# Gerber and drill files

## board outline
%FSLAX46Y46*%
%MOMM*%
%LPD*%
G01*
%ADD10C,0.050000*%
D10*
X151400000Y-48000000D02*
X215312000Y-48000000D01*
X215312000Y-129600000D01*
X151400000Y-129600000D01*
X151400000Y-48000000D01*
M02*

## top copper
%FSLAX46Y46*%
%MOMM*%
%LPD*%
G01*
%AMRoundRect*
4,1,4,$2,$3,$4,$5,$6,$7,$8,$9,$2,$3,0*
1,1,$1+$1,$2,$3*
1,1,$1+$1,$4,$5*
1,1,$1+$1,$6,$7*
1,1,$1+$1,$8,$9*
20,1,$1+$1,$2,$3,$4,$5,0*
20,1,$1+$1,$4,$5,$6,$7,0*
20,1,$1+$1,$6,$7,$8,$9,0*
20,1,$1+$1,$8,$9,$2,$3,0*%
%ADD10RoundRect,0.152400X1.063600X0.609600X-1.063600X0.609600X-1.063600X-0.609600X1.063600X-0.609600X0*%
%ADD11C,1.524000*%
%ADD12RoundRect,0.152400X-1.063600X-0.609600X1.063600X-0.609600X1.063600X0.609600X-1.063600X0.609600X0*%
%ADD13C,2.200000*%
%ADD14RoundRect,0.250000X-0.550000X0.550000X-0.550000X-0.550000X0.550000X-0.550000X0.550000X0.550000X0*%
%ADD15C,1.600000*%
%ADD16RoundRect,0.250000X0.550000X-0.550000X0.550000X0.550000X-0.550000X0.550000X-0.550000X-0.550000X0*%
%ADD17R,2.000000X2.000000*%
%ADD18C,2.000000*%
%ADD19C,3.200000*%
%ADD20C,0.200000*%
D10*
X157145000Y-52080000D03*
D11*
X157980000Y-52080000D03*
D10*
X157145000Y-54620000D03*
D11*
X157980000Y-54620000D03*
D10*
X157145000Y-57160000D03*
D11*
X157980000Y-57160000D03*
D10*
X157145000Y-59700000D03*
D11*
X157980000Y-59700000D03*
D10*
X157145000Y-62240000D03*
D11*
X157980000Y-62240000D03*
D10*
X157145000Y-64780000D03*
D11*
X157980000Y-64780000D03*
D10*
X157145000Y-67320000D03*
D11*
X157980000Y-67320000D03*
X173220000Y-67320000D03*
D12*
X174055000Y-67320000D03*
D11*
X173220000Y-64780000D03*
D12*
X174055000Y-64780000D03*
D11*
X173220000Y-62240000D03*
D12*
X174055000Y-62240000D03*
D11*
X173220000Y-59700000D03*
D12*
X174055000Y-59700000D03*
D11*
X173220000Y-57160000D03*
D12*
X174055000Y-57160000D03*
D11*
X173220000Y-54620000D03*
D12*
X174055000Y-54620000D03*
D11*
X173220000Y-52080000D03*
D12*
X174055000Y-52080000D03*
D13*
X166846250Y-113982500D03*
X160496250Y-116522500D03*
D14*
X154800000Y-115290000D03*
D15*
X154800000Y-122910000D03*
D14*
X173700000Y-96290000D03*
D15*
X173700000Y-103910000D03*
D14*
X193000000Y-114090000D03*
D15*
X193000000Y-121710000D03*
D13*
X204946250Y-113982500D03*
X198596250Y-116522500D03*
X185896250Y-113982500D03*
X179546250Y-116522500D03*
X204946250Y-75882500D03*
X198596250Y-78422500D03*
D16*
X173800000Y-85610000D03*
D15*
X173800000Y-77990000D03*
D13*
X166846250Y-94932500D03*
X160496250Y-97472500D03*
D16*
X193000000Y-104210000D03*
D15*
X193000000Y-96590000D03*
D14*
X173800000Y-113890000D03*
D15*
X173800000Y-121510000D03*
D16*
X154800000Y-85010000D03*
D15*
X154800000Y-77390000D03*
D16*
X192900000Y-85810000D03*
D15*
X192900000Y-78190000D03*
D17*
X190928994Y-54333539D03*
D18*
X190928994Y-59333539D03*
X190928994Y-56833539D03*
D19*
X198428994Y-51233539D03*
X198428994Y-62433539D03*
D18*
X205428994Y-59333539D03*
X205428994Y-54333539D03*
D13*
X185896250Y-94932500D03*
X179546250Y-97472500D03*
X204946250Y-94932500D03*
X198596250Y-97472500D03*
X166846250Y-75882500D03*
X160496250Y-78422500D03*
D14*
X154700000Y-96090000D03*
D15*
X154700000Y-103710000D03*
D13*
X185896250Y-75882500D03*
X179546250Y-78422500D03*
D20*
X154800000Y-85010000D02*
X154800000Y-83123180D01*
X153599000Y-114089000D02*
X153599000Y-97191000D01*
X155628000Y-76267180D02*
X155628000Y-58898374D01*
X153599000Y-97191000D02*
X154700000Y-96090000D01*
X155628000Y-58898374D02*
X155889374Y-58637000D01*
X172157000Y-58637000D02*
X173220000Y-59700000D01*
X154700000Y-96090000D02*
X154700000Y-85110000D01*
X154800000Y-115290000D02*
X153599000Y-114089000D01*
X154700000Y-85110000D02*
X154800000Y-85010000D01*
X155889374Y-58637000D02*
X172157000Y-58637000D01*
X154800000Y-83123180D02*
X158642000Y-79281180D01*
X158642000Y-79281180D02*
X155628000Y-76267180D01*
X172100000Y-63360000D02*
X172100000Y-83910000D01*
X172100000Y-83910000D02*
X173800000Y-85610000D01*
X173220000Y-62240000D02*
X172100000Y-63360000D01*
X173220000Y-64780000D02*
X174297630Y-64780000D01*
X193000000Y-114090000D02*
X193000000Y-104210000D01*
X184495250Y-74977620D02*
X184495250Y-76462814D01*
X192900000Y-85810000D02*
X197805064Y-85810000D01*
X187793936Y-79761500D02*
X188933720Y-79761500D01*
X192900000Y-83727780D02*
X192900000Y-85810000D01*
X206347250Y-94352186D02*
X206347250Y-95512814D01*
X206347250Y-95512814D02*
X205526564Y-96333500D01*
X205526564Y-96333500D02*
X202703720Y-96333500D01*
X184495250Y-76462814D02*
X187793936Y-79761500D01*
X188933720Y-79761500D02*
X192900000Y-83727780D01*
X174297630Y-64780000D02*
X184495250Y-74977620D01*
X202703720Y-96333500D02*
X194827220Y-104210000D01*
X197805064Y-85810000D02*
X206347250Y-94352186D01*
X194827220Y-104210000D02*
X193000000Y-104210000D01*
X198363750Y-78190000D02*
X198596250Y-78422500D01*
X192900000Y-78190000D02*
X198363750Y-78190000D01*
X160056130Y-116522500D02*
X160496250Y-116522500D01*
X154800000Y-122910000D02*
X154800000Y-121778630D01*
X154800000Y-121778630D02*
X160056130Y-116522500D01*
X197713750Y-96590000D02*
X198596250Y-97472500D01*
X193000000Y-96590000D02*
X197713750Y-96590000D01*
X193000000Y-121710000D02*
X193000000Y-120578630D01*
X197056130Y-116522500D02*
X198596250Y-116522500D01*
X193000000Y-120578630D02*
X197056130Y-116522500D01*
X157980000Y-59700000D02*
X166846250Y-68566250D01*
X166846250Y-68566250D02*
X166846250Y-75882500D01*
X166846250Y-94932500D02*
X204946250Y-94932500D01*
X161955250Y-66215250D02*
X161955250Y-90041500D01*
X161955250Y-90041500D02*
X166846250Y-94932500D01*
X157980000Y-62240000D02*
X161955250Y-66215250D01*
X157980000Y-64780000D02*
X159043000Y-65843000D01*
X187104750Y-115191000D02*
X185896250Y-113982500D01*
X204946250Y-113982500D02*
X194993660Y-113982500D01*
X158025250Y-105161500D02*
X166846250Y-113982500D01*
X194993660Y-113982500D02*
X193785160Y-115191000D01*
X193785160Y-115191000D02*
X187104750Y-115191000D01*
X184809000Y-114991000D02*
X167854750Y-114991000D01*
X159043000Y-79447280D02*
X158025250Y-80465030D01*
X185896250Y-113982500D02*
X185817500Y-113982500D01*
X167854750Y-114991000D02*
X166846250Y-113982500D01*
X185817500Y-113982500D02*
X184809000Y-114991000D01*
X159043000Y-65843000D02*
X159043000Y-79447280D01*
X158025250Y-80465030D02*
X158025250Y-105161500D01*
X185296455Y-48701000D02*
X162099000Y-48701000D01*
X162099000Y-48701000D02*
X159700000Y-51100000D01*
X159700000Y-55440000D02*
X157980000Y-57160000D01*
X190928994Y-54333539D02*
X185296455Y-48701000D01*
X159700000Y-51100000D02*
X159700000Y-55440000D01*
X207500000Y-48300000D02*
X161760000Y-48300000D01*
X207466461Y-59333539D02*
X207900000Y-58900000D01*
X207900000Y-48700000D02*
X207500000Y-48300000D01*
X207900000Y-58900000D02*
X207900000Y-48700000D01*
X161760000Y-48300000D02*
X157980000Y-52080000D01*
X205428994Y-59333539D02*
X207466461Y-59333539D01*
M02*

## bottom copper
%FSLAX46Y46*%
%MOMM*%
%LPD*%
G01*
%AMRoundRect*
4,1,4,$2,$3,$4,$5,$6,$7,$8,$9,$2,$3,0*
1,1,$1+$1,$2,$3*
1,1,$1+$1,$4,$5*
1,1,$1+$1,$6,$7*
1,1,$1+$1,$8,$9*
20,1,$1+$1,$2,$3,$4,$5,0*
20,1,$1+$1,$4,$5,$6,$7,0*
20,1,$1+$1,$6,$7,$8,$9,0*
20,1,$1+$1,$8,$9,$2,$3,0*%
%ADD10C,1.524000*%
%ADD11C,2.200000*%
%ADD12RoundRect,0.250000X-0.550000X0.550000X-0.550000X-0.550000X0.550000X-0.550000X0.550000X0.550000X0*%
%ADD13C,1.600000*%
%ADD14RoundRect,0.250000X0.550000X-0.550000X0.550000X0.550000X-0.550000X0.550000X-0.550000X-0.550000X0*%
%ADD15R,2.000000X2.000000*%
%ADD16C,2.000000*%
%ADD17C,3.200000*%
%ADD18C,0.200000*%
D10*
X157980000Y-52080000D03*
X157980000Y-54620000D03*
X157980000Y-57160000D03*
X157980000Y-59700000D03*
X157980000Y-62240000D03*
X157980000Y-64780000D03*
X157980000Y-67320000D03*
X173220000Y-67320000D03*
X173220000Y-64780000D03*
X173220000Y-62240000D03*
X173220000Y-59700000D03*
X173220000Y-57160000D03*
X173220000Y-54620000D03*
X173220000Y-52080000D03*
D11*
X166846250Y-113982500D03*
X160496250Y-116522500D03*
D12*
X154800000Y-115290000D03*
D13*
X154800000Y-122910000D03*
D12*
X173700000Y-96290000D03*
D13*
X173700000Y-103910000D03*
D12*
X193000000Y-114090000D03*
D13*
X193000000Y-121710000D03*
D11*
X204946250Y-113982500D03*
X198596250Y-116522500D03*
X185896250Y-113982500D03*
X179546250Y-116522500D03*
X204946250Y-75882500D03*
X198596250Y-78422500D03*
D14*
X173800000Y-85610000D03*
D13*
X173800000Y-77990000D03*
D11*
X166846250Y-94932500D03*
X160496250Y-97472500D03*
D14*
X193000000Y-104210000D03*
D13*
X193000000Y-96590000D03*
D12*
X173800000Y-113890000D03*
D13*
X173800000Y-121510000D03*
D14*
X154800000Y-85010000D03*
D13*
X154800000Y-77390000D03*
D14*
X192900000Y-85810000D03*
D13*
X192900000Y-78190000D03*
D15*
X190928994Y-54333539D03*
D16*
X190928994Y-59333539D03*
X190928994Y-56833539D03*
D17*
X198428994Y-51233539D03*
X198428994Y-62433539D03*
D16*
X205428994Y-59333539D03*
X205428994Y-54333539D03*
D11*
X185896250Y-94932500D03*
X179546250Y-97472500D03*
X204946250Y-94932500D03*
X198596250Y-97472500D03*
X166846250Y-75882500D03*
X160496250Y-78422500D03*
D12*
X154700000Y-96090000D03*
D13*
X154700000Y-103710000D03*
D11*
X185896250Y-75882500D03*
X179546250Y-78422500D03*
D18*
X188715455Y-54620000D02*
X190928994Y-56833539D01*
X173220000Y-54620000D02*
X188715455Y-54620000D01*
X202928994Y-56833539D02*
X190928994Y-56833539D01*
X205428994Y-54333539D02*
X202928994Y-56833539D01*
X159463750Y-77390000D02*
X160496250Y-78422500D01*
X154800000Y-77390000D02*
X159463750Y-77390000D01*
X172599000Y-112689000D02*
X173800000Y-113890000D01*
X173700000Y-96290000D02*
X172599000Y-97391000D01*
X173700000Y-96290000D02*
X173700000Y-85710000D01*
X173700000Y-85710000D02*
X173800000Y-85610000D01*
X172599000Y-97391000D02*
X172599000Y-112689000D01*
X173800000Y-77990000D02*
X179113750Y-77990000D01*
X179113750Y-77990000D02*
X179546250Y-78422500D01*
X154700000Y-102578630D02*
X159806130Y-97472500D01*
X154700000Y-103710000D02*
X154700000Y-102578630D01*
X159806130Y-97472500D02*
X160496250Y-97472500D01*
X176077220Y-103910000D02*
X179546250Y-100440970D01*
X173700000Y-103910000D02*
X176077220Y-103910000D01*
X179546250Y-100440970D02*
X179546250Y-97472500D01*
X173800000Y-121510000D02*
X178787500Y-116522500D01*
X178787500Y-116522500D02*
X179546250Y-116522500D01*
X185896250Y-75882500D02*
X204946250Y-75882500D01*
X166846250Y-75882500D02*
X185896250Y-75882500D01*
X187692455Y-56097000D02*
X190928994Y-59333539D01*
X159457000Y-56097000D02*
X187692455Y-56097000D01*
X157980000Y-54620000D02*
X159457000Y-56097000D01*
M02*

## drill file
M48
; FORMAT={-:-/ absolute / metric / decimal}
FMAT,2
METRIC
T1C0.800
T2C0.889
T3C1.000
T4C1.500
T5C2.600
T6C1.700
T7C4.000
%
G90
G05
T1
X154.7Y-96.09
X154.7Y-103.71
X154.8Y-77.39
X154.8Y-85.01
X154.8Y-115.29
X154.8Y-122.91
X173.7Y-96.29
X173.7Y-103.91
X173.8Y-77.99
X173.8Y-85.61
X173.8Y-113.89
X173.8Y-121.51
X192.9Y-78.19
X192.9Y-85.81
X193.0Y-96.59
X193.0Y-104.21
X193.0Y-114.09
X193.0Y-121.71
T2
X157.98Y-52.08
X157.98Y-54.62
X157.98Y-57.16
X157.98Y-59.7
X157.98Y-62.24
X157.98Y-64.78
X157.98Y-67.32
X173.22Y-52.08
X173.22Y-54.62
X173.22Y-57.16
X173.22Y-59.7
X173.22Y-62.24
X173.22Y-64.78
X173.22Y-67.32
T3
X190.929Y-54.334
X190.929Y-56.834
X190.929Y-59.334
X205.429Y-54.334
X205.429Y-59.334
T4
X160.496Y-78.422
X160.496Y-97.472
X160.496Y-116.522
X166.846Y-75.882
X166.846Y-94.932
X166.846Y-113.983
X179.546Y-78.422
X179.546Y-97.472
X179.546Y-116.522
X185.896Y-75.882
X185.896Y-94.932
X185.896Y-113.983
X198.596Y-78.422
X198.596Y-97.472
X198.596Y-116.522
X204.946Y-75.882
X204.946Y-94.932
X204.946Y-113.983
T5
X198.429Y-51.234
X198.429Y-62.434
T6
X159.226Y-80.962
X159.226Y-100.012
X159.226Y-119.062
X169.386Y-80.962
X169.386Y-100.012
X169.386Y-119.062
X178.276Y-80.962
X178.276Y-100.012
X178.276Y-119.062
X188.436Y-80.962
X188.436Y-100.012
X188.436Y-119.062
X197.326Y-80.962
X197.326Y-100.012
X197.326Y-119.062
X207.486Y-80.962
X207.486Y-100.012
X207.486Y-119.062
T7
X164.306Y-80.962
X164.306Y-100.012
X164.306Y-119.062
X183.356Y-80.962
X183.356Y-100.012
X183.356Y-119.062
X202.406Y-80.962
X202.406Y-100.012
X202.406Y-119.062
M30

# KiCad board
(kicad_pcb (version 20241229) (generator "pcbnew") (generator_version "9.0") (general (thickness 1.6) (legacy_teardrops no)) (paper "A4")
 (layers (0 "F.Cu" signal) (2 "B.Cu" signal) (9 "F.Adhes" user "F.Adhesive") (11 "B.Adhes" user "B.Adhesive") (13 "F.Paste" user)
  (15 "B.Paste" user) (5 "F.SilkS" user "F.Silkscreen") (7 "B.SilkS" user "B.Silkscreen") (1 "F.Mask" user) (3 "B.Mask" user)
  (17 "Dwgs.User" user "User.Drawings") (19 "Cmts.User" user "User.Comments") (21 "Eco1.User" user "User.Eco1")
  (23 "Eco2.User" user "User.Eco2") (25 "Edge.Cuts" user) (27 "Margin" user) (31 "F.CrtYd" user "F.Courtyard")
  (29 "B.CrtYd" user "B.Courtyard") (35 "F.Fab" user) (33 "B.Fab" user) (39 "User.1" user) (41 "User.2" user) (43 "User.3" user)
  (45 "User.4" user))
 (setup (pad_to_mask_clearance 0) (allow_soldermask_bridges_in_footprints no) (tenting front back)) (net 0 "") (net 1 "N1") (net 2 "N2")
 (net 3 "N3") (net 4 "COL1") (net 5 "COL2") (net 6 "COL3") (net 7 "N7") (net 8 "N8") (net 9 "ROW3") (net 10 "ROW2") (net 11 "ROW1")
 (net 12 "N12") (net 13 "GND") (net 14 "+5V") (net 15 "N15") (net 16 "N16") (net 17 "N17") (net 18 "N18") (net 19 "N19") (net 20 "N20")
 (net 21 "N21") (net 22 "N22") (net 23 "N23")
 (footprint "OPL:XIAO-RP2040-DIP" (layer "F.Cu") (at 165.6 59.7)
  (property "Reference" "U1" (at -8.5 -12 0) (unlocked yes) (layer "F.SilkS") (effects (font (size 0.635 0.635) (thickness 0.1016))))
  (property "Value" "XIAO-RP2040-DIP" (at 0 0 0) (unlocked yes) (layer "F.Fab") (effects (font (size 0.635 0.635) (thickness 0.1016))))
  (pad "1" smd roundrect (at -8.455 -7.62 180) (size 2.432 1.524) (layers "F.Cu" "F.Mask") (roundrect_rratio 0.1) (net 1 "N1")
   (thermal_bridge_angle 45))
  (pad "1" thru_hole circle (at -7.62 -7.62 180) (size 1.524 1.524) (drill 0.889) (layers "*.Cu" "*.Mask") (remove_unused_layers no)
   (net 1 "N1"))
  (pad "2" smd roundrect (at -8.455 -5.08 180) (size 2.432 1.524) (layers "F.Cu" "F.Mask") (roundrect_rratio 0.1) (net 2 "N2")
   (thermal_bridge_angle 45))
  (pad "2" thru_hole circle (at -7.62 -5.08 180) (size 1.524 1.524) (drill 0.889) (layers "*.Cu" "*.Mask") (remove_unused_layers no)
   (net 2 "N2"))
  (pad "3" smd roundrect (at -8.455 -2.54 180) (size 2.432 1.524) (layers "F.Cu" "F.Mask") (roundrect_rratio 0.1) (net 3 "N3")
   (thermal_bridge_angle 45))
  (pad "3" thru_hole circle (at -7.62 -2.54 180) (size 1.524 1.524) (drill 0.889) (layers "*.Cu" "*.Mask") (remove_unused_layers no)
   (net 3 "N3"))
  (pad "4" smd roundrect (at -8.455 0 180) (size 2.432 1.524) (layers "F.Cu" "F.Mask") (roundrect_rratio 0.1) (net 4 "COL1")
   (thermal_bridge_angle 45))
  (pad "4" thru_hole circle (at -7.62 0 180) (size 1.524 1.524) (drill 0.889) (layers "*.Cu" "*.Mask") (remove_unused_layers no)
   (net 4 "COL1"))
  (pad "5" smd roundrect (at -8.455 2.54 180) (size 2.432 1.524) (layers "F.Cu" "F.Mask") (roundrect_rratio 0.1) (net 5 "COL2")
   (thermal_bridge_angle 45))
  (pad "5" thru_hole circle (at -7.62 2.54 180) (size 1.524 1.524) (drill 0.889) (layers "*.Cu" "*.Mask") (remove_unused_layers no)
   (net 5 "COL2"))
  (pad "6" smd roundrect (at -8.455 5.08 180) (size 2.432 1.524) (layers "F.Cu" "F.Mask") (roundrect_rratio 0.1) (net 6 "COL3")
   (thermal_bridge_angle 45))
  (pad "6" thru_hole circle (at -7.62 5.08 180) (size 1.524 1.524) (drill 0.889) (layers "*.Cu" "*.Mask") (remove_unused_layers no)
   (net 6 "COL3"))
  (pad "7" smd roundrect (at -8.455 7.62 180) (size 2.432 1.524) (layers "F.Cu" "F.Mask") (roundrect_rratio 0.1) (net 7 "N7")
   (thermal_bridge_angle 45))
  (pad "7" thru_hole circle (at -7.62 7.62 180) (size 1.524 1.524) (drill 0.889) (layers "*.Cu" "*.Mask") (remove_unused_layers no)
   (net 7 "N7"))
  (pad "8" thru_hole circle (at 7.62 7.62) (size 1.524 1.524) (drill 0.889) (layers "*.Cu" "*.Mask") (remove_unused_layers no) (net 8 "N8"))
  (pad "8" smd roundrect (at 8.455 7.62) (size 2.432 1.524) (layers "F.Cu" "F.Mask") (roundrect_rratio 0.1) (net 8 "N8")
   (thermal_bridge_angle 45))
  (pad "9" thru_hole circle (at 7.62 5.08) (size 1.524 1.524) (drill 0.889) (layers "*.Cu" "*.Mask") (remove_unused_layers no)
   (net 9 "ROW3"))
  (pad "9" smd roundrect (at 8.455 5.08) (size 2.432 1.524) (layers "F.Cu" "F.Mask") (roundrect_rratio 0.1) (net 9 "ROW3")
   (thermal_bridge_angle 45))
  (pad "10" thru_hole circle (at 7.62 2.54) (size 1.524 1.524) (drill 0.889) (layers "*.Cu" "*.Mask") (remove_unused_layers no)
   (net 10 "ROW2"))
  (pad "10" smd roundrect (at 8.455 2.54) (size 2.432 1.524) (layers "F.Cu" "F.Mask") (roundrect_rratio 0.1) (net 10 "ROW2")
   (thermal_bridge_angle 45))
  (pad "11" thru_hole circle (at 7.62 0) (size 1.524 1.524) (drill 0.889) (layers "*.Cu" "*.Mask") (remove_unused_layers no) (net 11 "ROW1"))
  (pad "11" smd roundrect (at 8.455 0) (size 2.432 1.524) (layers "F.Cu" "F.Mask") (roundrect_rratio 0.1) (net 11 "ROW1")
   (thermal_bridge_angle 45))
  (pad "12" thru_hole circle (at 7.62 -2.54) (size 1.524 1.524) (drill 0.889) (layers "*.Cu" "*.Mask") (remove_unused_layers no)
   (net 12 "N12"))
  (pad "12" smd roundrect (at 8.455 -2.54) (size 2.432 1.524) (layers "F.Cu" "F.Mask") (roundrect_rratio 0.1) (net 12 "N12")
   (thermal_bridge_angle 45))
  (pad "13" thru_hole circle (at 7.62 -5.08) (size 1.524 1.524) (drill 0.889) (layers "*.Cu" "*.Mask") (remove_unused_layers no)
   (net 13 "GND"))
  (pad "13" smd roundrect (at 8.455 -5.08) (size 2.432 1.524) (layers "F.Cu" "F.Mask") (roundrect_rratio 0.1) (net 13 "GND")
   (thermal_bridge_angle 45))
  (pad "14" thru_hole circle (at 7.62 -7.62) (size 1.524 1.524) (drill 0.889) (layers "*.Cu" "*.Mask") (remove_unused_layers no)
   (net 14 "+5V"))
  (pad "14" smd roundrect (at 8.455 -7.62) (size 2.432 1.524) (layers "F.Cu" "F.Mask") (roundrect_rratio 0.1) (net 14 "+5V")
   (thermal_bridge_angle 45)))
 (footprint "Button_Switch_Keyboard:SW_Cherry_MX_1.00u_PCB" (layer "F.Cu") (at 166.84625 113.9825)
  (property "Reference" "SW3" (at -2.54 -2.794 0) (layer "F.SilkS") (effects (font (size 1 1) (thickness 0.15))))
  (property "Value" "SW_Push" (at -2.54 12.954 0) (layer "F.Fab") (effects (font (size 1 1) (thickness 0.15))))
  (pad "" np_thru_hole circle (at -7.62 5.08) (size 1.7 1.7) (drill 1.7) (layers "*.Cu" "*.Mask"))
  (pad "" np_thru_hole circle (at -2.54 5.08) (size 4 4) (drill 4) (layers "*.Cu" "*.Mask"))
  (pad "" np_thru_hole circle (at 2.54 5.08) (size 1.7 1.7) (drill 1.7) (layers "*.Cu" "*.Mask"))
  (pad "1" thru_hole circle (at 0 0) (size 2.2 2.2) (drill 1.5) (layers "*.Cu" "*.Mask") (remove_unused_layers no) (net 6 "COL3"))
  (pad "2" thru_hole circle (at -6.35 2.54) (size 2.2 2.2) (drill 1.5) (layers "*.Cu" "*.Mask") (remove_unused_layers no) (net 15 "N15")))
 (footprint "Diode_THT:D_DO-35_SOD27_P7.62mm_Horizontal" (layer "F.Cu") (at 154.8 115.29 -90)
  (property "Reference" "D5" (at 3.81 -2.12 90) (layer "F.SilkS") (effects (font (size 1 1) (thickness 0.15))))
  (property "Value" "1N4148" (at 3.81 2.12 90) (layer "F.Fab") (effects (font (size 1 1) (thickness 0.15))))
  (pad "1" thru_hole roundrect (at 0 0 270) (size 1.6 1.6) (drill 0.8) (layers "*.Cu" "*.Mask") (remove_unused_layers no)
   (roundrect_rratio 0.15625) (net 11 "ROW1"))
  (pad "2" thru_hole circle (at 7.62 0 270) (size 1.6 1.6) (drill 0.8) (layers "*.Cu" "*.Mask") (remove_unused_layers no) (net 15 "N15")))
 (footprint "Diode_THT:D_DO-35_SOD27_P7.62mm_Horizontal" (layer "F.Cu") (at 173.7 96.29 -90)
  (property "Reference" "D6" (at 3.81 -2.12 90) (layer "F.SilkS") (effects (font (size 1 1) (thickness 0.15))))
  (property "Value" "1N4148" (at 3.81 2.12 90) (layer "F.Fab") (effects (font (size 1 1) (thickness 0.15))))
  (pad "1" thru_hole roundrect (at 0 0 270) (size 1.6 1.6) (drill 0.8) (layers "*.Cu" "*.Mask") (remove_unused_layers no)
   (roundrect_rratio 0.15625) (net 10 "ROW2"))
  (pad "2" thru_hole circle (at 7.62 0 270) (size 1.6 1.6) (drill 0.8) (layers "*.Cu" "*.Mask") (remove_unused_layers no) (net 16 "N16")))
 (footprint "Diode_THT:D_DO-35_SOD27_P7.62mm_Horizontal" (layer "F.Cu") (at 193 114.09 -90)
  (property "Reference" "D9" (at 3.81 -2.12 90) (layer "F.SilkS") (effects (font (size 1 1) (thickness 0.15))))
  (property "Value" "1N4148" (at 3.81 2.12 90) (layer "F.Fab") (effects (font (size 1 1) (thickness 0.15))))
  (pad "1" thru_hole roundrect (at 0 0 270) (size 1.6 1.6) (drill 0.8) (layers "*.Cu" "*.Mask") (remove_unused_layers no)
   (roundrect_rratio 0.15625) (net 9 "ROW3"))
  (pad "2" thru_hole circle (at 7.62 0 270) (size 1.6 1.6) (drill 0.8) (layers "*.Cu" "*.Mask") (remove_unused_layers no) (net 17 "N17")))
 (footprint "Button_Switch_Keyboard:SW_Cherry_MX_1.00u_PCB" (layer "F.Cu") (at 204.94625 113.9825)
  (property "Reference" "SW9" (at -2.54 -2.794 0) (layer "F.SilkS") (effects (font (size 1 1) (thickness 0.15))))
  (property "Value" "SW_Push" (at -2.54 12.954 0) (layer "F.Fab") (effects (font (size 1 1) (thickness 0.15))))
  (pad "" np_thru_hole circle (at -7.62 5.08) (size 1.7 1.7) (drill 1.7) (layers "*.Cu" "*.Mask"))
  (pad "" np_thru_hole circle (at -2.54 5.08) (size 4 4) (drill 4) (layers "*.Cu" "*.Mask"))
  (pad "" np_thru_hole circle (at 2.54 5.08) (size 1.7 1.7) (drill 1.7) (layers "*.Cu" "*.Mask"))
  (pad "1" thru_hole circle (at 0 0) (size 2.2 2.2) (drill 1.5) (layers "*.Cu" "*.Mask") (remove_unused_layers no) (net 6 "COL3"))
  (pad "2" thru_hole circle (at -6.35 2.54) (size 2.2 2.2) (drill 1.5) (layers "*.Cu" "*.Mask") (remove_unused_layers no) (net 17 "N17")))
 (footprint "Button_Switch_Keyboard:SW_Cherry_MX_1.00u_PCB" (layer "F.Cu") (at 185.89625 113.9825)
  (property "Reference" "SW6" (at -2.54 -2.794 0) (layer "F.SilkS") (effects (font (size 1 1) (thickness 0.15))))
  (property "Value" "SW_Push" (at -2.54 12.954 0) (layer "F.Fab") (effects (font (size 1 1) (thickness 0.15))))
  (pad "" np_thru_hole circle (at -7.62 5.08) (size 1.7 1.7) (drill 1.7) (layers "*.Cu" "*.Mask"))
  (pad "" np_thru_hole circle (at -2.54 5.08) (size 4 4) (drill 4) (layers "*.Cu" "*.Mask"))
  (pad "" np_thru_hole circle (at 2.54 5.08) (size 1.7 1.7) (drill 1.7) (layers "*.Cu" "*.Mask"))
  (pad "1" thru_hole circle (at 0 0) (size 2.2 2.2) (drill 1.5) (layers "*.Cu" "*.Mask") (remove_unused_layers no) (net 6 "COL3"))
  (pad "2" thru_hole circle (at -6.35 2.54) (size 2.2 2.2) (drill 1.5) (layers "*.Cu" "*.Mask") (remove_unused_layers no) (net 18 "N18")))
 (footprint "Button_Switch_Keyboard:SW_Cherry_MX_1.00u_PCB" (layer "F.Cu") (at 204.94625 75.8825)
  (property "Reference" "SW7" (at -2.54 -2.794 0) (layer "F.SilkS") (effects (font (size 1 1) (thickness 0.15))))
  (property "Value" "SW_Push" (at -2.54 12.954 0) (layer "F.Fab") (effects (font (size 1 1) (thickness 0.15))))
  (pad "" np_thru_hole circle (at -7.62 5.08) (size 1.7 1.7) (drill 1.7) (layers "*.Cu" "*.Mask"))
  (pad "" np_thru_hole circle (at -2.54 5.08) (size 4 4) (drill 4) (layers "*.Cu" "*.Mask"))
  (pad "" np_thru_hole circle (at 2.54 5.08) (size 1.7 1.7) (drill 1.7) (layers "*.Cu" "*.Mask"))
  (pad "1" thru_hole circle (at 0 0) (size 2.2 2.2) (drill 1.5) (layers "*.Cu" "*.Mask") (remove_unused_layers no) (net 4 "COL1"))
  (pad "2" thru_hole circle (at -6.35 2.54) (size 2.2 2.2) (drill 1.5) (layers "*.Cu" "*.Mask") (remove_unused_layers no) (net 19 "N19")))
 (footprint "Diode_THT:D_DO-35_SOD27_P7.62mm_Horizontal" (layer "F.Cu") (at 173.8 85.61 90)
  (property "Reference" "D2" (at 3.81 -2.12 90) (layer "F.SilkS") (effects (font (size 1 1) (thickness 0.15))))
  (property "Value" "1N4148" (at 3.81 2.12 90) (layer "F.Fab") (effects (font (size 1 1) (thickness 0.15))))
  (pad "1" thru_hole roundrect (at 0 0 90) (size 1.6 1.6) (drill 0.8) (layers "*.Cu" "*.Mask") (remove_unused_layers no)
   (roundrect_rratio 0.15625) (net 10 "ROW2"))
  (pad "2" thru_hole circle (at 7.62 0 90) (size 1.6 1.6) (drill 0.8) (layers "*.Cu" "*.Mask") (remove_unused_layers no) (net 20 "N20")))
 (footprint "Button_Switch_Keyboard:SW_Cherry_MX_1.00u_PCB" (layer "F.Cu") (at 166.84625 94.9325)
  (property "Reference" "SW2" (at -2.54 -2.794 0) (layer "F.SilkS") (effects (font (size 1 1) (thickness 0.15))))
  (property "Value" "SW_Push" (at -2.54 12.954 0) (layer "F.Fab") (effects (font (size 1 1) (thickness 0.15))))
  (pad "" np_thru_hole circle (at -7.62 5.08) (size 1.7 1.7) (drill 1.7) (layers "*.Cu" "*.Mask"))
  (pad "" np_thru_hole circle (at -2.54 5.08) (size 4 4) (drill 4) (layers "*.Cu" "*.Mask"))
  (pad "" np_thru_hole circle (at 2.54 5.08) (size 1.7 1.7) (drill 1.7) (layers "*.Cu" "*.Mask"))
  (pad "1" thru_hole circle (at 0 0) (size 2.2 2.2) (drill 1.5) (layers "*.Cu" "*.Mask") (remove_unused_layers no) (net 5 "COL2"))
  (pad "2" thru_hole circle (at -6.35 2.54) (size 2.2 2.2) (drill 1.5) (layers "*.Cu" "*.Mask") (remove_unused_layers no) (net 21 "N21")))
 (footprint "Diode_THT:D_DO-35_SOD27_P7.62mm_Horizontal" (layer "F.Cu") (at 193 104.21 90)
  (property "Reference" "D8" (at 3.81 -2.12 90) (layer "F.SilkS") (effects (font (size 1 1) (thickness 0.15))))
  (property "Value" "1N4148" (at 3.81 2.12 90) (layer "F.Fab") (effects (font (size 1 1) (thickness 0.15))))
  (pad "1" thru_hole roundrect (at 0 0 90) (size 1.6 1.6) (drill 0.8) (layers "*.Cu" "*.Mask") (remove_unused_layers no)
   (roundrect_rratio 0.15625) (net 9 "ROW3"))
  (pad "2" thru_hole circle (at 7.62 0 90) (size 1.6 1.6) (drill 0.8) (layers "*.Cu" "*.Mask") (remove_unused_layers no) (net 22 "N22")))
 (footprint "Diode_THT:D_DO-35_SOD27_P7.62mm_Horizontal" (layer "F.Cu") (at 173.8 113.89 -90)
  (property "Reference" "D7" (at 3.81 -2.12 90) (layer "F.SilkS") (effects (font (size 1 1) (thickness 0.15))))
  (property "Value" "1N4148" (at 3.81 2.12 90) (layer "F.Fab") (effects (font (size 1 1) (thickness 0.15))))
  (pad "1" thru_hole roundrect (at 0 0 270) (size 1.6 1.6) (drill 0.8) (layers "*.Cu" "*.Mask") (remove_unused_layers no)
   (roundrect_rratio 0.15625) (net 10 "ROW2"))
  (pad "2" thru_hole circle (at 7.62 0 270) (size 1.6 1.6) (drill 0.8) (layers "*.Cu" "*.Mask") (remove_unused_layers no) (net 18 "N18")))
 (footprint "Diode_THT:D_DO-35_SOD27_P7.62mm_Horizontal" (layer "F.Cu") (at 154.8 85.01 90)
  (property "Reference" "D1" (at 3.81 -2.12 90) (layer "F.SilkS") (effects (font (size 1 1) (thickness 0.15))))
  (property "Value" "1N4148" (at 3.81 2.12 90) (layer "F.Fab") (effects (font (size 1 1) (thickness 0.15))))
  (pad "1" thru_hole roundrect (at 0 0 90) (size 1.6 1.6) (drill 0.8) (layers "*.Cu" "*.Mask") (remove_unused_layers no)
   (roundrect_rratio 0.15625) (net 11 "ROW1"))
  (pad "2" thru_hole circle (at 7.62 0 90) (size 1.6 1.6) (drill 0.8) (layers "*.Cu" "*.Mask") (remove_unused_layers no) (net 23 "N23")))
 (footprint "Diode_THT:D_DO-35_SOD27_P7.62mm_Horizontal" (layer "F.Cu") (at 192.9 85.81 90)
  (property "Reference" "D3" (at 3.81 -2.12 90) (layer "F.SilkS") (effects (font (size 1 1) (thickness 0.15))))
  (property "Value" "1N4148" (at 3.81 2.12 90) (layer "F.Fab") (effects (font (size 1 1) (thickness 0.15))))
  (pad "1" thru_hole roundrect (at 0 0 90) (size 1.6 1.6) (drill 0.8) (layers "*.Cu" "*.Mask") (remove_unused_layers no)
   (roundrect_rratio 0.15625) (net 9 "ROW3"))
  (pad "2" thru_hole circle (at 7.62 0 90) (size 1.6 1.6) (drill 0.8) (layers "*.Cu" "*.Mask") (remove_unused_layers no) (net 19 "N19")))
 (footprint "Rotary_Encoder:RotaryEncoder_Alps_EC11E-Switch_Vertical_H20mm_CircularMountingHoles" (layer "F.Cu") (at 190.928994 54.333539)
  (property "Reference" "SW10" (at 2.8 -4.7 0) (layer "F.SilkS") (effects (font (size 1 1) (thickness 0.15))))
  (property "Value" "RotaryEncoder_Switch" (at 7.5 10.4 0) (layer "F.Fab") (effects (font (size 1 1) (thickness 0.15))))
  (pad "A" thru_hole rect (at 0 0) (size 2 2) (drill 1) (layers "*.Cu" "*.Mask") (remove_unused_layers no) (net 3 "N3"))
  (pad "B" thru_hole circle (at 0 5) (size 2 2) (drill 1) (layers "*.Cu" "*.Mask") (remove_unused_layers no) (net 2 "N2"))
  (pad "C" thru_hole circle (at 0 2.5) (size 2 2) (drill 1) (layers "*.Cu" "*.Mask") (remove_unused_layers no) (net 13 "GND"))
  (pad "MP" thru_hole circle (at 7.5 -3.1) (size 3.2 3.2) (drill 2.6) (layers "*.Cu" "*.Mask") (remove_unused_layers no))
  (pad "MP" thru_hole circle (at 7.5 8.1) (size 3.2 3.2) (drill 2.6) (layers "*.Cu" "*.Mask") (remove_unused_layers no))
  (pad "S1" thru_hole circle (at 14.5 5) (size 2 2) (drill 1) (layers "*.Cu" "*.Mask") (remove_unused_layers no) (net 1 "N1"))
  (pad "S2" thru_hole circle (at 14.5 0) (size 2 2) (drill 1) (layers "*.Cu" "*.Mask") (remove_unused_layers no) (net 13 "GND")))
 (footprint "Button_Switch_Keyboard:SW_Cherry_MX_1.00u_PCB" (layer "F.Cu") (at 185.89625 94.9325)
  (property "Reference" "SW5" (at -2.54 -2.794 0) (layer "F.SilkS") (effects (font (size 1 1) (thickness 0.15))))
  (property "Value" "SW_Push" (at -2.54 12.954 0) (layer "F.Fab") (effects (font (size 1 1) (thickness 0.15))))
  (pad "" np_thru_hole circle (at -7.62 5.08) (size 1.7 1.7) (drill 1.7) (layers "*.Cu" "*.Mask"))
  (pad "" np_thru_hole circle (at -2.54 5.08) (size 4 4) (drill 4) (layers "*.Cu" "*.Mask"))
  (pad "" np_thru_hole circle (at 2.54 5.08) (size 1.7 1.7) (drill 1.7) (layers "*.Cu" "*.Mask"))
  (pad "1" thru_hole circle (at 0 0) (size 2.2 2.2) (drill 1.5) (layers "*.Cu" "*.Mask") (remove_unused_layers no) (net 5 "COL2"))
  (pad "2" thru_hole circle (at -6.35 2.54) (size 2.2 2.2) (drill 1.5) (layers "*.Cu" "*.Mask") (remove_unused_layers no) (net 16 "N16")))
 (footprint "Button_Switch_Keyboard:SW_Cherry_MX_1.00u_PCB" (layer "F.Cu") (at 204.94625 94.9325)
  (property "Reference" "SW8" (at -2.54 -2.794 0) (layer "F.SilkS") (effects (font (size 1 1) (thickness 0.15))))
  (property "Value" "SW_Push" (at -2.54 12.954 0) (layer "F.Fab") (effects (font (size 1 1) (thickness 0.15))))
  (pad "" np_thru_hole circle (at -7.62 5.08) (size 1.7 1.7) (drill 1.7) (layers "*.Cu" "*.Mask"))
  (pad "" np_thru_hole circle (at -2.54 5.08) (size 4 4) (drill 4) (layers "*.Cu" "*.Mask"))
  (pad "" np_thru_hole circle (at 2.54 5.08) (size 1.7 1.7) (drill 1.7) (layers "*.Cu" "*.Mask"))
  (pad "1" thru_hole circle (at 0 0) (size 2.2 2.2) (drill 1.5) (layers "*.Cu" "*.Mask") (remove_unused_layers no) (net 5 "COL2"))
  (pad "2" thru_hole circle (at -6.35 2.54) (size 2.2 2.2) (drill 1.5) (layers "*.Cu" "*.Mask") (remove_unused_layers no) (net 22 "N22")))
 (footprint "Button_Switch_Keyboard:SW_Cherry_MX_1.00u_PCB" (layer "F.Cu") (at 166.84625 75.8825)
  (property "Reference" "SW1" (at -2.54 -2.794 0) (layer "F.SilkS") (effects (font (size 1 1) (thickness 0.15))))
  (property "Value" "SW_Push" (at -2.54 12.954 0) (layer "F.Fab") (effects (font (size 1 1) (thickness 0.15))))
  (pad "" np_thru_hole circle (at -7.62 5.08) (size 1.7 1.7) (drill 1.7) (layers "*.Cu" "*.Mask"))
  (pad "" np_thru_hole circle (at -2.54 5.08) (size 4 4) (drill 4) (layers "*.Cu" "*.Mask"))
  (pad "" np_thru_hole circle (at 2.54 5.08) (size 1.7 1.7) (drill 1.7) (layers "*.Cu" "*.Mask"))
  (pad "1" thru_hole circle (at 0 0) (size 2.2 2.2) (drill 1.5) (layers "*.Cu" "*.Mask") (remove_unused_layers no) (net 4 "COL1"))
  (pad "2" thru_hole circle (at -6.35 2.54) (size 2.2 2.2) (drill 1.5) (layers "*.Cu" "*.Mask") (remove_unused_layers no) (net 23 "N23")))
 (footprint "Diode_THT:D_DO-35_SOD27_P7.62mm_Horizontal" (layer "F.Cu") (at 154.7 96.09 -90)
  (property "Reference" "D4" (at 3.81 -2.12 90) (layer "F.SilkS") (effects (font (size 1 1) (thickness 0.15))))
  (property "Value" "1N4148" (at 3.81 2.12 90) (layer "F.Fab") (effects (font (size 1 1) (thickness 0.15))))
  (pad "1" thru_hole roundrect (at 0 0 270) (size 1.6 1.6) (drill 0.8) (layers "*.Cu" "*.Mask") (remove_unused_layers no)
   (roundrect_rratio 0.15625) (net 11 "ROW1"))
  (pad "2" thru_hole circle (at 7.62 0 270) (size 1.6 1.6) (drill 0.8) (layers "*.Cu" "*.Mask") (remove_unused_layers no) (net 21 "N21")))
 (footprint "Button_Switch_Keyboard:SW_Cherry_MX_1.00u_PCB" (layer "F.Cu") (at 185.89625 75.8825)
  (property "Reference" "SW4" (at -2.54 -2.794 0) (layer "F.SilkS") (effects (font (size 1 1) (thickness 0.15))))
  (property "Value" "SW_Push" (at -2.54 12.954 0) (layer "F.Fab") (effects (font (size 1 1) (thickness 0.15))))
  (pad "" np_thru_hole circle (at -7.62 5.08) (size 1.7 1.7) (drill 1.7) (layers "*.Cu" "*.Mask"))
  (pad "" np_thru_hole circle (at -2.54 5.08) (size 4 4) (drill 4) (layers "*.Cu" "*.Mask"))
  (pad "" np_thru_hole circle (at 2.54 5.08) (size 1.7 1.7) (drill 1.7) (layers "*.Cu" "*.Mask"))
  (pad "1" thru_hole circle (at 0 0) (size 2.2 2.2) (drill 1.5) (layers "*.Cu" "*.Mask") (remove_unused_layers no) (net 4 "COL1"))
  (pad "2" thru_hole circle (at -6.35 2.54) (size 2.2 2.2) (drill 1.5) (layers "*.Cu" "*.Mask") (remove_unused_layers no) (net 20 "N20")))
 (gr_rect (start 151.4 48) (end 215.312 129.6) (stroke (width 0.05) (type default)) (fill no) (layer "Edge.Cuts"))
 (segment (start 188.715455 54.62) (end 190.928994 56.833539) (width 0.2) (layer "B.Cu") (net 13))
 (segment (start 173.22 54.62) (end 188.715455 54.62) (width 0.2) (layer "B.Cu") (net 13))
 (segment (start 202.928994 56.833539) (end 190.928994 56.833539) (width 0.2) (layer "B.Cu") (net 13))
 (segment (start 205.428994 54.333539) (end 202.928994 56.833539) (width 0.2) (layer "B.Cu") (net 13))
 (segment (start 154.8 85.01) (end 154.8 83.12318) (width 0.2) (layer "F.Cu") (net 11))
 (segment (start 153.599 114.089) (end 153.599 97.191) (width 0.2) (layer "F.Cu") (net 11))
 (segment (start 155.628 76.26718) (end 155.628 58.898374) (width 0.2) (layer "F.Cu") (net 11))
 (segment (start 153.599 97.191) (end 154.7 96.09) (width 0.2) (layer "F.Cu") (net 11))
 (segment (start 155.628 58.898374) (end 155.889374 58.637) (width 0.2) (layer "F.Cu") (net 11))
 (segment (start 172.157 58.637) (end 173.22 59.7) (width 0.2) (layer "F.Cu") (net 11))
 (segment (start 154.7 96.09) (end 154.7 85.11) (width 0.2) (layer "F.Cu") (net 11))
 (segment (start 154.8 115.29) (end 153.599 114.089) (width 0.2) (layer "F.Cu") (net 11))
 (segment (start 154.7 85.11) (end 154.8 85.01) (width 0.2) (layer "F.Cu") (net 11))
 (segment (start 155.889374 58.637) (end 172.157 58.637) (width 0.2) (layer "F.Cu") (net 11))
 (segment (start 154.8 83.12318) (end 158.642 79.28118) (width 0.2) (layer "F.Cu") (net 11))
 (segment (start 158.642 79.28118) (end 155.628 76.26718) (width 0.2) (layer "F.Cu") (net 11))
 (segment (start 159.46375 77.39) (end 160.49625 78.4225) (width 0.2) (layer "B.Cu") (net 23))
 (segment (start 154.8 77.39) (end 159.46375 77.39) (width 0.2) (layer "B.Cu") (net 23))
 (segment (start 172.1 63.36) (end 172.1 83.91) (width 0.2) (layer "F.Cu") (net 10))
 (segment (start 172.1 83.91) (end 173.8 85.61) (width 0.2) (layer "F.Cu") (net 10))
 (segment (start 173.22 62.24) (end 172.1 63.36) (width 0.2) (layer "F.Cu") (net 10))
 (segment (start 172.599 112.689) (end 173.8 113.89) (width 0.2) (layer "B.Cu") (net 10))
 (segment (start 173.7 96.29) (end 172.599 97.391) (width 0.2) (layer "B.Cu") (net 10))
 (segment (start 173.7 96.29) (end 173.7 85.71) (width 0.2) (layer "B.Cu") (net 10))
 (segment (start 173.7 85.71) (end 173.8 85.61) (width 0.2) (layer "B.Cu") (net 10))
 (segment (start 172.599 97.391) (end 172.599 112.689) (width 0.2) (layer "B.Cu") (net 10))
 (segment (start 173.8 77.99) (end 179.11375 77.99) (width 0.2) (layer "B.Cu") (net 20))
 (segment (start 179.11375 77.99) (end 179.54625 78.4225) (width 0.2) (layer "B.Cu") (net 20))
 (segment (start 173.22 64.78) (end 174.29763 64.78) (width 0.2) (layer "F.Cu") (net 9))
 (segment (start 193 114.09) (end 193 104.21) (width 0.2) (layer "F.Cu") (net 9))
 (segment (start 184.49525 74.97762) (end 184.49525 76.462814) (width 0.2) (layer "F.Cu") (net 9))
 (segment (start 192.9 85.81) (end 197.805064 85.81) (width 0.2) (layer "F.Cu") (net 9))
 (segment (start 187.793936 79.7615) (end 188.93372 79.7615) (width 0.2) (layer "F.Cu") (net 9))
 (segment (start 192.9 83.72778) (end 192.9 85.81) (width 0.2) (layer "F.Cu") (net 9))
 (segment (start 206.34725 94.352186) (end 206.34725 95.512814) (width 0.2) (layer "F.Cu") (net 9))
 (segment (start 206.34725 95.512814) (end 205.526564 96.3335) (width 0.2) (layer "F.Cu") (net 9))
 (segment (start 205.526564 96.3335) (end 202.70372 96.3335) (width 0.2) (layer "F.Cu") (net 9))
 (segment (start 184.49525 76.462814) (end 187.793936 79.7615) (width 0.2) (layer "F.Cu") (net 9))
 (segment (start 188.93372 79.7615) (end 192.9 83.72778) (width 0.2) (layer "F.Cu") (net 9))
 (segment (start 174.29763 64.78) (end 184.49525 74.97762) (width 0.2) (layer "F.Cu") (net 9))
 (segment (start 202.70372 96.3335) (end 194.82722 104.21) (width 0.2) (layer "F.Cu") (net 9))
 (segment (start 197.805064 85.81) (end 206.34725 94.352186) (width 0.2) (layer "F.Cu") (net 9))
 (segment (start 194.82722 104.21) (end 193 104.21) (width 0.2) (layer "F.Cu") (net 9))
 (segment (start 198.36375 78.19) (end 198.59625 78.4225) (width 0.2) (layer "F.Cu") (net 19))
 (segment (start 192.9 78.19) (end 198.36375 78.19) (width 0.2) (layer "F.Cu") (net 19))
 (segment (start 154.7 102.57863) (end 159.80613 97.4725) (width 0.2) (layer "B.Cu") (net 21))
 (segment (start 154.7 103.71) (end 154.7 102.57863) (width 0.2) (layer "B.Cu") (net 21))
 (segment (start 159.80613 97.4725) (end 160.49625 97.4725) (width 0.2) (layer "B.Cu") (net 21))
 (segment (start 160.05613 116.5225) (end 160.49625 116.5225) (width 0.2) (layer "F.Cu") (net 15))
 (segment (start 154.8 122.91) (end 154.8 121.77863) (width 0.2) (layer "F.Cu") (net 15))
 (segment (start 154.8 121.77863) (end 160.05613 116.5225) (width 0.2) (layer "F.Cu") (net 15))
 (segment (start 176.07722 103.91) (end 179.54625 100.44097) (width 0.2) (layer "B.Cu") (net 16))
 (segment (start 173.7 103.91) (end 176.07722 103.91) (width 0.2) (layer "B.Cu") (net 16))
 (segment (start 179.54625 100.44097) (end 179.54625 97.4725) (width 0.2) (layer "B.Cu") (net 16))
 (segment (start 173.8 121.51) (end 178.7875 116.5225) (width 0.2) (layer "B.Cu") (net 18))
 (segment (start 178.7875 116.5225) (end 179.54625 116.5225) (width 0.2) (layer "B.Cu") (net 18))
 (segment (start 197.71375 96.59) (end 198.59625 97.4725) (width 0.2) (layer "F.Cu") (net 22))
 (segment (start 193 96.59) (end 197.71375 96.59) (width 0.2) (layer "F.Cu") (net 22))
 (segment (start 193 121.71) (end 193 120.57863) (width 0.2) (layer "F.Cu") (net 17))
 (segment (start 197.05613 116.5225) (end 198.59625 116.5225) (width 0.2) (layer "F.Cu") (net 17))
 (segment (start 193 120.57863) (end 197.05613 116.5225) (width 0.2) (layer "F.Cu") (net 17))
 (segment (start 157.98 59.7) (end 166.84625 68.56625) (width 0.2) (layer "F.Cu") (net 4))
 (segment (start 166.84625 68.56625) (end 166.84625 75.8825) (width 0.2) (layer "F.Cu") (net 4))
 (segment (start 185.89625 75.8825) (end 204.94625 75.8825) (width 0.2) (layer "B.Cu") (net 4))
 (segment (start 166.84625 75.8825) (end 185.89625 75.8825) (width 0.2) (layer "B.Cu") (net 4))
 (segment (start 166.84625 94.9325) (end 204.94625 94.9325) (width 0.2) (layer "F.Cu") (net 5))
 (segment (start 161.95525 66.21525) (end 161.95525 90.0415) (width 0.2) (layer "F.Cu") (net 5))
 (segment (start 161.95525 90.0415) (end 166.84625 94.9325) (width 0.2) (layer "F.Cu") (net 5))
 (segment (start 157.98 62.24) (end 161.95525 66.21525) (width 0.2) (layer "F.Cu") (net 5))
 (segment (start 157.98 64.78) (end 159.043 65.843) (width 0.2) (layer "F.Cu") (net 6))
 (segment (start 187.10475 115.191) (end 185.89625 113.9825) (width 0.2) (layer "F.Cu") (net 6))
 (segment (start 204.94625 113.9825) (end 194.99366 113.9825) (width 0.2) (layer "F.Cu") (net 6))
 (segment (start 158.02525 105.1615) (end 166.84625 113.9825) (width 0.2) (layer "F.Cu") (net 6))
 (segment (start 194.99366 113.9825) (end 193.78516 115.191) (width 0.2) (layer "F.Cu") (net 6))
 (segment (start 193.78516 115.191) (end 187.10475 115.191) (width 0.2) (layer "F.Cu") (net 6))
 (segment (start 184.809 114.991) (end 167.85475 114.991) (width 0.2) (layer "F.Cu") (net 6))
 (segment (start 159.043 79.44728) (end 158.02525 80.46503) (width 0.2) (layer "F.Cu") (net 6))
 (segment (start 185.89625 113.9825) (end 185.8175 113.9825) (width 0.2) (layer "F.Cu") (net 6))
 (segment (start 167.85475 114.991) (end 166.84625 113.9825) (width 0.2) (layer "F.Cu") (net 6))
 (segment (start 185.8175 113.9825) (end 184.809 114.991) (width 0.2) (layer "F.Cu") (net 6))
 (segment (start 159.043 65.843) (end 159.043 79.44728) (width 0.2) (layer "F.Cu") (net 6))
 (segment (start 158.02525 80.46503) (end 158.02525 105.1615) (width 0.2) (layer "F.Cu") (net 6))
 (segment (start 187.692455 56.097) (end 190.928994 59.333539) (width 0.2) (layer "B.Cu") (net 2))
 (segment (start 159.457 56.097) (end 187.692455 56.097) (width 0.2) (layer "B.Cu") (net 2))
 (segment (start 157.98 54.62) (end 159.457 56.097) (width 0.2) (layer "B.Cu") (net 2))
 (segment (start 185.296455 48.701) (end 162.099 48.701) (width 0.2) (layer "F.Cu") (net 3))
 (segment (start 162.099 48.701) (end 159.7 51.1) (width 0.2) (layer "F.Cu") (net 3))
 (segment (start 159.7 55.44) (end 157.98 57.16) (width 0.2) (layer "F.Cu") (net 3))
 (segment (start 190.928994 54.333539) (end 185.296455 48.701) (width 0.2) (layer "F.Cu") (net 3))
 (segment (start 159.7 51.1) (end 159.7 55.44) (width 0.2) (layer "F.Cu") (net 3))
 (segment (start 207.5 48.3) (end 161.76 48.3) (width 0.2) (layer "F.Cu") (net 1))
 (segment (start 207.466461 59.333539) (end 207.9 58.9) (width 0.2) (layer "F.Cu") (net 1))
 (segment (start 207.9 48.7) (end 207.5 48.3) (width 0.2) (layer "F.Cu") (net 1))
 (segment (start 207.9 58.9) (end 207.9 48.7) (width 0.2) (layer "F.Cu") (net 1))
 (segment (start 161.76 48.3) (end 157.98 52.08) (width 0.2) (layer "F.Cu") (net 1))
 (segment (start 205.428994 59.333539) (end 207.466461 59.333539) (width 0.2) (layer "F.Cu") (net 1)))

